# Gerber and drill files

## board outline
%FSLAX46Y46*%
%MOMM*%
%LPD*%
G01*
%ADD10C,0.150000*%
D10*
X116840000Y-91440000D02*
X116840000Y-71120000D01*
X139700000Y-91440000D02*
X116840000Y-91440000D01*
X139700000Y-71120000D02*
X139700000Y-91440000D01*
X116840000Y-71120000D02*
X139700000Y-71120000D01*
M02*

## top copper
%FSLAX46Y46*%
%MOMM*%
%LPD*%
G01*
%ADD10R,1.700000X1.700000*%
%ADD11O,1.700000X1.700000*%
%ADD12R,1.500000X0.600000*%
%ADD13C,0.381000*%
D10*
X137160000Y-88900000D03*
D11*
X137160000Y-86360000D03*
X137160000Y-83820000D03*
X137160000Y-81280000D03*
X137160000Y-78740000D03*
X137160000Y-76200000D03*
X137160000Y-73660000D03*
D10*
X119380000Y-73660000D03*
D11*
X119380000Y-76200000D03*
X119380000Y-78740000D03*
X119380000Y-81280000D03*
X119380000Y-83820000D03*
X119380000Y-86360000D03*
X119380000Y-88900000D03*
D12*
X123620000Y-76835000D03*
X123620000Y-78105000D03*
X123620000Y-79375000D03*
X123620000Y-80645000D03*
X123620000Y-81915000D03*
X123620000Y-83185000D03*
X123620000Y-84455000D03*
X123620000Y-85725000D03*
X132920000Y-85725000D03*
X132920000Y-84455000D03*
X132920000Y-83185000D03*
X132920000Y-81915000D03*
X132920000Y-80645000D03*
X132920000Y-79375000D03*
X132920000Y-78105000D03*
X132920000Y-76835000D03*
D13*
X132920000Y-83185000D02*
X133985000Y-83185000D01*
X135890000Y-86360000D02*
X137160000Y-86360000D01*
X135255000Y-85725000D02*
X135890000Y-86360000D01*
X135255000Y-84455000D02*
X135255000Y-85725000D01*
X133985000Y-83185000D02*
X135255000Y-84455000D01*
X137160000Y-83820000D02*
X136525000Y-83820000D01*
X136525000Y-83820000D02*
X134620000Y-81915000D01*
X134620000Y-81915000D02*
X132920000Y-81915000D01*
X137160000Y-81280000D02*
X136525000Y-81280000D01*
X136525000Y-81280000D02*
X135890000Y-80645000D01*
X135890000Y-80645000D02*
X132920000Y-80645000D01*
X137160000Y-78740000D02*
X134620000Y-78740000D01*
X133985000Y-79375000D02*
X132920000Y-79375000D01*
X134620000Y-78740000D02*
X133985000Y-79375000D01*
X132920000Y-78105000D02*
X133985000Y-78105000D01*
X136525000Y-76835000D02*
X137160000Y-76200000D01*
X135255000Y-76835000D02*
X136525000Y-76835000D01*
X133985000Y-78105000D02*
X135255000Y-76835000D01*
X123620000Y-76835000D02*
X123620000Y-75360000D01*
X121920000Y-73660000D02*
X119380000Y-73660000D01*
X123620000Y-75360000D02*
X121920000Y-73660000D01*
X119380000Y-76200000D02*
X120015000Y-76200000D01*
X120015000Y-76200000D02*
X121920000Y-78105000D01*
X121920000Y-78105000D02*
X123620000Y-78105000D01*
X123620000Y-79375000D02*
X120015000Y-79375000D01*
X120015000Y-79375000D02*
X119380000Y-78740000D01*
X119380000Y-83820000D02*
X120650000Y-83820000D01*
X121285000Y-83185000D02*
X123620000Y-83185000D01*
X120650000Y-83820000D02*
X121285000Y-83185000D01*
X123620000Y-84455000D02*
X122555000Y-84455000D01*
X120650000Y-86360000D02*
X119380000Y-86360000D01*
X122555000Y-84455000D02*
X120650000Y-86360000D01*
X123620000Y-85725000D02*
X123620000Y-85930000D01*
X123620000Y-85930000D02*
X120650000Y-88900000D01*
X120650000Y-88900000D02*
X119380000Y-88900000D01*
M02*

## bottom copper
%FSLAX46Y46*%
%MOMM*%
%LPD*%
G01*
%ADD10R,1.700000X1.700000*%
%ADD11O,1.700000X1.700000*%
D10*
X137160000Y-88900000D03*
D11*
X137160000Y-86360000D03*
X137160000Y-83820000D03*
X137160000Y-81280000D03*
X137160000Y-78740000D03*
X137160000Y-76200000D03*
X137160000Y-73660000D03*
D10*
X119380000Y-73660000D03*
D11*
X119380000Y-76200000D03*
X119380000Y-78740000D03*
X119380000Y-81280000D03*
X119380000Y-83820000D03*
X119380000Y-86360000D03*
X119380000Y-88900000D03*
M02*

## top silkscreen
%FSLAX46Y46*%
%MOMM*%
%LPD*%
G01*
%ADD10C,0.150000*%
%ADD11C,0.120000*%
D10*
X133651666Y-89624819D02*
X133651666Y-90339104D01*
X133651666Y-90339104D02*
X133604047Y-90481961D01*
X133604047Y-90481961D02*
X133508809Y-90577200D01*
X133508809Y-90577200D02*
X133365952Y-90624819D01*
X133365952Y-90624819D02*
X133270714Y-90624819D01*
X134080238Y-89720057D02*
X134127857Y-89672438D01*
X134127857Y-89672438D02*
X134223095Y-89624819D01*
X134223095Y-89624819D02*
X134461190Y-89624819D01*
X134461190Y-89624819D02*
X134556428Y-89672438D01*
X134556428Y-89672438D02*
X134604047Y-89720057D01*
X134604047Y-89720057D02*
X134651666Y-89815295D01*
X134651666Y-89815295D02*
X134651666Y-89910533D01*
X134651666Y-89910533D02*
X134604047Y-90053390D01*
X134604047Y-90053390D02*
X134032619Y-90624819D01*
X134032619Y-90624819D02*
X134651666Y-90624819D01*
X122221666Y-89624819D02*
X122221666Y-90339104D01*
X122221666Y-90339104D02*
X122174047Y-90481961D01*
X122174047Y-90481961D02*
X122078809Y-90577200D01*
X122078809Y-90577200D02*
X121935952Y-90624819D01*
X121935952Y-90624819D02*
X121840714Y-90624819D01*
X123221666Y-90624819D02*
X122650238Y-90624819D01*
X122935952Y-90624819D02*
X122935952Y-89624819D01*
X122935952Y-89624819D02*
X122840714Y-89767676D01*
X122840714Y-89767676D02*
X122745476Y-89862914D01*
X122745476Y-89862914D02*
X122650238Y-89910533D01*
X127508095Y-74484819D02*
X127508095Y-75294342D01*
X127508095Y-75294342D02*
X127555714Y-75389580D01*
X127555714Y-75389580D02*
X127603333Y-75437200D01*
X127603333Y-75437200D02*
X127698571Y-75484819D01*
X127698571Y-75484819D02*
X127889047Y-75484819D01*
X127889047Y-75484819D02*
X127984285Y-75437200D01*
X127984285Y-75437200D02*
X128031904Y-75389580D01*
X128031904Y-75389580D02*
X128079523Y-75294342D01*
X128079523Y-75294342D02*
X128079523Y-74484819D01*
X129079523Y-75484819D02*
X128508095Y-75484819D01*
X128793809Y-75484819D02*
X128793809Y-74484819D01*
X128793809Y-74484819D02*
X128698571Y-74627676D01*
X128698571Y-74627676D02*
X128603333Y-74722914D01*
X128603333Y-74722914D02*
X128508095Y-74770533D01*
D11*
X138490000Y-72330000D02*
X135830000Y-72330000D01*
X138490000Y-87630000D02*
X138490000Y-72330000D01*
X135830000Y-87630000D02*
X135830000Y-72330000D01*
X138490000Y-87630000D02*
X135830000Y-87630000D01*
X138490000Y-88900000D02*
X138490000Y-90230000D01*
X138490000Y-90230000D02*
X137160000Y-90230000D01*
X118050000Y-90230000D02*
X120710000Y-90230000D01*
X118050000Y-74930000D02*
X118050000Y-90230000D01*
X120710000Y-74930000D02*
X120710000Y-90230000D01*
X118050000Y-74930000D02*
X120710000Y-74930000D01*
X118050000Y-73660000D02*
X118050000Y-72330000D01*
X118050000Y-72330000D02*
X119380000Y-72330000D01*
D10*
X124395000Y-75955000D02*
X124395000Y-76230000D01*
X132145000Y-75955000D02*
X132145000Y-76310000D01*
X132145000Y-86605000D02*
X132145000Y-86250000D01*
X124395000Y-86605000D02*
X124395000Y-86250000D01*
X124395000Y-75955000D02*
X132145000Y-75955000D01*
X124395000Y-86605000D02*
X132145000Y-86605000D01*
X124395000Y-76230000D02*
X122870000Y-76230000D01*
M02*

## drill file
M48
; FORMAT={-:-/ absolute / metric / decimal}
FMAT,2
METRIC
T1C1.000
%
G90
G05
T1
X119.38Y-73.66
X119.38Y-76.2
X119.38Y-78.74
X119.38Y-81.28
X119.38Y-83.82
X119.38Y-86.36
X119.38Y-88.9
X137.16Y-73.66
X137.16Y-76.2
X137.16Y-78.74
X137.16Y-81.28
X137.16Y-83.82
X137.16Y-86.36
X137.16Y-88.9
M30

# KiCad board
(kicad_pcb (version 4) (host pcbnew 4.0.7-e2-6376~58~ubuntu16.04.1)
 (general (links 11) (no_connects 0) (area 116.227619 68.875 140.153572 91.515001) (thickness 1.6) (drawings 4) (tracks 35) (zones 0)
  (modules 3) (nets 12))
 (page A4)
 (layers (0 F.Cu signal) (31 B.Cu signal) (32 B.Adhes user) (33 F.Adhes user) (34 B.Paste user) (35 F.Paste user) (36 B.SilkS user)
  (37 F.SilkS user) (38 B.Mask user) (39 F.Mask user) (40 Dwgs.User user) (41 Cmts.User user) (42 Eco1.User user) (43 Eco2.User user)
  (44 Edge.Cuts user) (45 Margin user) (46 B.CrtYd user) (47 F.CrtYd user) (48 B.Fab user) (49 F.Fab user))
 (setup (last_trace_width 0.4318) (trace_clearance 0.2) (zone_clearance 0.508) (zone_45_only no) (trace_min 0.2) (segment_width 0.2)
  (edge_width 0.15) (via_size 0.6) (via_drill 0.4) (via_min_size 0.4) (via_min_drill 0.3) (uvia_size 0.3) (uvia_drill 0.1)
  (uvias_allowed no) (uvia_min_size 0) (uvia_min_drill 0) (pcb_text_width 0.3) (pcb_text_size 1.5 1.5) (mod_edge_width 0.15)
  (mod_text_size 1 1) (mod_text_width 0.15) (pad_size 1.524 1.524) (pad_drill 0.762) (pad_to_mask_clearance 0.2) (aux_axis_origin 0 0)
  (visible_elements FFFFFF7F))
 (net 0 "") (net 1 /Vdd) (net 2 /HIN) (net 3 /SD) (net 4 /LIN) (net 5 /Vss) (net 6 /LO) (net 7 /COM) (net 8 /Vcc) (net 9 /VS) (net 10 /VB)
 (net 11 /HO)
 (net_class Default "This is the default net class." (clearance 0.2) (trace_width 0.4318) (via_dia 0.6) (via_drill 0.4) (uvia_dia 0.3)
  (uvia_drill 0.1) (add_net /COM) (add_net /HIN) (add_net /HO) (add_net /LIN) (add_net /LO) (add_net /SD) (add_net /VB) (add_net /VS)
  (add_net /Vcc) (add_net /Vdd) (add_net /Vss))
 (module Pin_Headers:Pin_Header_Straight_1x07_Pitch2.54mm (layer F.Cu) (at 137.16 88.9 180)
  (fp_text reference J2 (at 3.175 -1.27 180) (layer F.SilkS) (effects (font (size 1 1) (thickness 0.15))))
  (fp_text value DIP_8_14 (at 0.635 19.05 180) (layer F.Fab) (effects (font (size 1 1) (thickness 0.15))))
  (fp_line (start -1.33 16.57) (end 1.33 16.57) (layer F.SilkS) (width 0.12))
  (fp_line (start -1.33 1.27) (end -1.33 16.57) (layer F.SilkS) (width 0.12))
  (fp_line (start 1.33 1.27) (end 1.33 16.57) (layer F.SilkS) (width 0.12))
  (fp_line (start -1.33 1.27) (end 1.33 1.27) (layer F.SilkS) (width 0.12))
  (fp_line (start -1.33 0) (end -1.33 -1.33) (layer F.SilkS) (width 0.12))
  (fp_line (start -1.33 -1.33) (end 0 -1.33) (layer F.SilkS) (width 0.12))
  (pad 1 thru_hole rect (at 0 0 180) (size 1.7 1.7) (drill 1) (layers *.Cu *.Mask))
  (pad 2 thru_hole oval (at 0 2.54 180) (size 1.7 1.7) (drill 1) (layers *.Cu *.Mask) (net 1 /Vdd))
  (pad 3 thru_hole oval (at 0 5.08 180) (size 1.7 1.7) (drill 1) (layers *.Cu *.Mask) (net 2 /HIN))
  (pad 4 thru_hole oval (at 0 7.62 180) (size 1.7 1.7) (drill 1) (layers *.Cu *.Mask) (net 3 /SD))
  (pad 5 thru_hole oval (at 0 10.16 180) (size 1.7 1.7) (drill 1) (layers *.Cu *.Mask) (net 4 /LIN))
  (pad 6 thru_hole oval (at 0 12.7 180) (size 1.7 1.7) (drill 1) (layers *.Cu *.Mask) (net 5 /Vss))
  (pad 7 thru_hole oval (at 0 15.24 180) (size 1.7 1.7) (drill 1) (layers *.Cu *.Mask)))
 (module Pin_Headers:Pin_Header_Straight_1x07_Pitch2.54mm (layer F.Cu) (at 119.38 73.66)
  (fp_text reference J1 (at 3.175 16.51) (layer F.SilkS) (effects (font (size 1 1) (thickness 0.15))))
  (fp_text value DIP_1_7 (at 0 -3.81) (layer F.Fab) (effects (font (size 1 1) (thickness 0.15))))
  (fp_line (start -1.33 16.57) (end 1.33 16.57) (layer F.SilkS) (width 0.12))
  (fp_line (start -1.33 1.27) (end -1.33 16.57) (layer F.SilkS) (width 0.12))
  (fp_line (start 1.33 1.27) (end 1.33 16.57) (layer F.SilkS) (width 0.12))
  (fp_line (start -1.33 1.27) (end 1.33 1.27) (layer F.SilkS) (width 0.12))
  (fp_line (start -1.33 0) (end -1.33 -1.33) (layer F.SilkS) (width 0.12))
  (fp_line (start -1.33 -1.33) (end 0 -1.33) (layer F.SilkS) (width 0.12))
  (pad 1 thru_hole rect (at 0 0) (size 1.7 1.7) (drill 1) (layers *.Cu *.Mask) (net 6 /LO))
  (pad 2 thru_hole oval (at 0 2.54) (size 1.7 1.7) (drill 1) (layers *.Cu *.Mask) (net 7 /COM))
  (pad 3 thru_hole oval (at 0 5.08) (size 1.7 1.7) (drill 1) (layers *.Cu *.Mask) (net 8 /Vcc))
  (pad 4 thru_hole oval (at 0 7.62) (size 1.7 1.7) (drill 1) (layers *.Cu *.Mask))
  (pad 5 thru_hole oval (at 0 10.16) (size 1.7 1.7) (drill 1) (layers *.Cu *.Mask) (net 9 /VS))
  (pad 6 thru_hole oval (at 0 12.7) (size 1.7 1.7) (drill 1) (layers *.Cu *.Mask) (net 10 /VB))
  (pad 7 thru_hole oval (at 0 15.24) (size 1.7 1.7) (drill 1) (layers *.Cu *.Mask) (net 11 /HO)))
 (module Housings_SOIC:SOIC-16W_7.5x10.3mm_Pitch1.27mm (layer F.Cu) (at 128.27 81.28)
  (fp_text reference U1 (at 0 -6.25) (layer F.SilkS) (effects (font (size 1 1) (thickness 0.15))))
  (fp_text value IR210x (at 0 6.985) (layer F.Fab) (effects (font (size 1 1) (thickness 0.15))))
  (fp_line (start -3.875 -5.325) (end -3.875 -5.05) (layer F.SilkS) (width 0.15))
  (fp_line (start 3.875 -5.325) (end 3.875 -4.97) (layer F.SilkS) (width 0.15))
  (fp_line (start 3.875 5.325) (end 3.875 4.97) (layer F.SilkS) (width 0.15))
  (fp_line (start -3.875 5.325) (end -3.875 4.97) (layer F.SilkS) (width 0.15))
  (fp_line (start -3.875 -5.325) (end 3.875 -5.325) (layer F.SilkS) (width 0.15))
  (fp_line (start -3.875 5.325) (end 3.875 5.325) (layer F.SilkS) (width 0.15))
  (fp_line (start -3.875 -5.05) (end -5.4 -5.05) (layer F.SilkS) (width 0.15))
  (pad 1 smd rect (at -4.65 -4.445) (size 1.5 0.6) (layers F.Cu F.Paste F.Mask) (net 6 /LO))
  (pad 2 smd rect (at -4.65 -3.175) (size 1.5 0.6) (layers F.Cu F.Paste F.Mask) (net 7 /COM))
  (pad 3 smd rect (at -4.65 -1.905) (size 1.5 0.6) (layers F.Cu F.Paste F.Mask) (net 8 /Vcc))
  (pad 4 smd rect (at -4.65 -0.635) (size 1.5 0.6) (layers F.Cu F.Paste F.Mask))
  (pad 5 smd rect (at -4.65 0.635) (size 1.5 0.6) (layers F.Cu F.Paste F.Mask))
  (pad 6 smd rect (at -4.65 1.905) (size 1.5 0.6) (layers F.Cu F.Paste F.Mask) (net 9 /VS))
  (pad 7 smd rect (at -4.65 3.175) (size 1.5 0.6) (layers F.Cu F.Paste F.Mask) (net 10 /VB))
  (pad 8 smd rect (at -4.65 4.445) (size 1.5 0.6) (layers F.Cu F.Paste F.Mask) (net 11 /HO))
  (pad 9 smd rect (at 4.65 4.445) (size 1.5 0.6) (layers F.Cu F.Paste F.Mask))
  (pad 10 smd rect (at 4.65 3.175) (size 1.5 0.6) (layers F.Cu F.Paste F.Mask))
  (pad 11 smd rect (at 4.65 1.905) (size 1.5 0.6) (layers F.Cu F.Paste F.Mask) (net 1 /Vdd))
  (pad 12 smd rect (at 4.65 0.635) (size 1.5 0.6) (layers F.Cu F.Paste F.Mask) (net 2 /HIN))
  (pad 13 smd rect (at 4.65 -0.635) (size 1.5 0.6) (layers F.Cu F.Paste F.Mask) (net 3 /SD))
  (pad 14 smd rect (at 4.65 -1.905) (size 1.5 0.6) (layers F.Cu F.Paste F.Mask) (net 4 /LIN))
  (pad 15 smd rect (at 4.65 -3.175) (size 1.5 0.6) (layers F.Cu F.Paste F.Mask) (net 5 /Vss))
  (pad 16 smd rect (at 4.65 -4.445) (size 1.5 0.6) (layers F.Cu F.Paste F.Mask)))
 (gr_line (start 116.84 91.44) (end 116.84 71.12) (angle 90) (layer Edge.Cuts) (width 0.15))
 (gr_line (start 139.7 91.44) (end 116.84 91.44) (angle 90) (layer Edge.Cuts) (width 0.15))
 (gr_line (start 139.7 71.12) (end 139.7 91.44) (angle 90) (layer Edge.Cuts) (width 0.15))
 (gr_line (start 116.84 71.12) (end 139.7 71.12) (angle 90) (layer Edge.Cuts) (width 0.15))
 (segment (start 132.92 83.185) (end 133.985 83.185) (width 0.381) (layer F.Cu) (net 1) (status 400000))
 (segment (start 135.89 86.36) (end 137.16 86.36) (width 0.381) (layer F.Cu) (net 1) (status 800000))
 (segment (start 135.255 85.725) (end 135.89 86.36) (width 0.381) (layer F.Cu) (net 1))
 (segment (start 135.255 84.455) (end 135.255 85.725) (width 0.381) (layer F.Cu) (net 1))
 (segment (start 133.985 83.185) (end 135.255 84.455) (width 0.381) (layer F.Cu) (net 1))
 (segment (start 137.16 83.82) (end 136.525 83.82) (width 0.381) (layer F.Cu) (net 2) (status C00000))
 (segment (start 136.525 83.82) (end 134.62 81.915) (width 0.381) (layer F.Cu) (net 2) (status 400000))
 (segment (start 134.62 81.915) (end 132.92 81.915) (width 0.381) (layer F.Cu) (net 2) (status 800000))
 (segment (start 137.16 81.28) (end 136.525 81.28) (width 0.381) (layer F.Cu) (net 3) (status C00000))
 (segment (start 136.525 81.28) (end 135.89 80.645) (width 0.381) (layer F.Cu) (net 3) (status 400000))
 (segment (start 135.89 80.645) (end 132.92 80.645) (width 0.381) (layer F.Cu) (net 3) (status 800000))
 (segment (start 137.16 78.74) (end 134.62 78.74) (width 0.381) (layer F.Cu) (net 4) (status 400000))
 (segment (start 133.985 79.375) (end 132.92 79.375) (width 0.381) (layer F.Cu) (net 4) (status 800000))
 (segment (start 134.62 78.74) (end 133.985 79.375) (width 0.381) (layer F.Cu) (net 4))
 (segment (start 132.92 78.105) (end 133.985 78.105) (width 0.381) (layer F.Cu) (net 5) (status 400000))
 (segment (start 136.525 76.835) (end 137.16 76.2) (width 0.381) (layer F.Cu) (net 5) (status 800000))
 (segment (start 135.255 76.835) (end 136.525 76.835) (width 0.381) (layer F.Cu) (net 5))
 (segment (start 133.985 78.105) (end 135.255 76.835) (width 0.381) (layer F.Cu) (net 5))
 (segment (start 123.62 76.835) (end 123.62 75.36) (width 0.381) (layer F.Cu) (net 6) (status 400000))
 (segment (start 121.92 73.66) (end 119.38 73.66) (width 0.381) (layer F.Cu) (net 6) (status 800000))
 (segment (start 123.62 75.36) (end 121.92 73.66) (width 0.381) (layer F.Cu) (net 6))
 (segment (start 119.38 76.2) (end 120.015 76.2) (width 0.381) (layer F.Cu) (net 7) (status C00000))
 (segment (start 120.015 76.2) (end 121.92 78.105) (width 0.381) (layer F.Cu) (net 7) (status 400000))
 (segment (start 121.92 78.105) (end 123.62 78.105) (width 0.381) (layer F.Cu) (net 7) (status 800000))
 (segment (start 123.62 79.375) (end 120.015 79.375) (width 0.381) (layer F.Cu) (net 8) (status 400000))
 (segment (start 120.015 79.375) (end 119.38 78.74) (width 0.381) (layer F.Cu) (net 8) (status 800000))
 (segment (start 119.38 83.82) (end 120.65 83.82) (width 0.381) (layer F.Cu) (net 9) (status 400000))
 (segment (start 121.285 83.185) (end 123.62 83.185) (width 0.381) (layer F.Cu) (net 9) (status 800000))
 (segment (start 120.65 83.82) (end 121.285 83.185) (width 0.381) (layer F.Cu) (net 9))
 (segment (start 123.62 84.455) (end 122.555 84.455) (width 0.381) (layer F.Cu) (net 10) (status 400000))
 (segment (start 120.65 86.36) (end 119.38 86.36) (width 0.381) (layer F.Cu) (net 10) (status 800000))
 (segment (start 122.555 84.455) (end 120.65 86.36) (width 0.381) (layer F.Cu) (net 10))
 (segment (start 123.62 85.725) (end 123.62 85.93) (width 0.381) (layer F.Cu) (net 11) (status C00000))
 (segment (start 123.62 85.93) (end 120.65 88.9) (width 0.381) (layer F.Cu) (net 11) (status 400000))
 (segment (start 120.65 88.9) (end 119.38 88.9) (width 0.381) (layer F.Cu) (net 11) (status 800000)))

